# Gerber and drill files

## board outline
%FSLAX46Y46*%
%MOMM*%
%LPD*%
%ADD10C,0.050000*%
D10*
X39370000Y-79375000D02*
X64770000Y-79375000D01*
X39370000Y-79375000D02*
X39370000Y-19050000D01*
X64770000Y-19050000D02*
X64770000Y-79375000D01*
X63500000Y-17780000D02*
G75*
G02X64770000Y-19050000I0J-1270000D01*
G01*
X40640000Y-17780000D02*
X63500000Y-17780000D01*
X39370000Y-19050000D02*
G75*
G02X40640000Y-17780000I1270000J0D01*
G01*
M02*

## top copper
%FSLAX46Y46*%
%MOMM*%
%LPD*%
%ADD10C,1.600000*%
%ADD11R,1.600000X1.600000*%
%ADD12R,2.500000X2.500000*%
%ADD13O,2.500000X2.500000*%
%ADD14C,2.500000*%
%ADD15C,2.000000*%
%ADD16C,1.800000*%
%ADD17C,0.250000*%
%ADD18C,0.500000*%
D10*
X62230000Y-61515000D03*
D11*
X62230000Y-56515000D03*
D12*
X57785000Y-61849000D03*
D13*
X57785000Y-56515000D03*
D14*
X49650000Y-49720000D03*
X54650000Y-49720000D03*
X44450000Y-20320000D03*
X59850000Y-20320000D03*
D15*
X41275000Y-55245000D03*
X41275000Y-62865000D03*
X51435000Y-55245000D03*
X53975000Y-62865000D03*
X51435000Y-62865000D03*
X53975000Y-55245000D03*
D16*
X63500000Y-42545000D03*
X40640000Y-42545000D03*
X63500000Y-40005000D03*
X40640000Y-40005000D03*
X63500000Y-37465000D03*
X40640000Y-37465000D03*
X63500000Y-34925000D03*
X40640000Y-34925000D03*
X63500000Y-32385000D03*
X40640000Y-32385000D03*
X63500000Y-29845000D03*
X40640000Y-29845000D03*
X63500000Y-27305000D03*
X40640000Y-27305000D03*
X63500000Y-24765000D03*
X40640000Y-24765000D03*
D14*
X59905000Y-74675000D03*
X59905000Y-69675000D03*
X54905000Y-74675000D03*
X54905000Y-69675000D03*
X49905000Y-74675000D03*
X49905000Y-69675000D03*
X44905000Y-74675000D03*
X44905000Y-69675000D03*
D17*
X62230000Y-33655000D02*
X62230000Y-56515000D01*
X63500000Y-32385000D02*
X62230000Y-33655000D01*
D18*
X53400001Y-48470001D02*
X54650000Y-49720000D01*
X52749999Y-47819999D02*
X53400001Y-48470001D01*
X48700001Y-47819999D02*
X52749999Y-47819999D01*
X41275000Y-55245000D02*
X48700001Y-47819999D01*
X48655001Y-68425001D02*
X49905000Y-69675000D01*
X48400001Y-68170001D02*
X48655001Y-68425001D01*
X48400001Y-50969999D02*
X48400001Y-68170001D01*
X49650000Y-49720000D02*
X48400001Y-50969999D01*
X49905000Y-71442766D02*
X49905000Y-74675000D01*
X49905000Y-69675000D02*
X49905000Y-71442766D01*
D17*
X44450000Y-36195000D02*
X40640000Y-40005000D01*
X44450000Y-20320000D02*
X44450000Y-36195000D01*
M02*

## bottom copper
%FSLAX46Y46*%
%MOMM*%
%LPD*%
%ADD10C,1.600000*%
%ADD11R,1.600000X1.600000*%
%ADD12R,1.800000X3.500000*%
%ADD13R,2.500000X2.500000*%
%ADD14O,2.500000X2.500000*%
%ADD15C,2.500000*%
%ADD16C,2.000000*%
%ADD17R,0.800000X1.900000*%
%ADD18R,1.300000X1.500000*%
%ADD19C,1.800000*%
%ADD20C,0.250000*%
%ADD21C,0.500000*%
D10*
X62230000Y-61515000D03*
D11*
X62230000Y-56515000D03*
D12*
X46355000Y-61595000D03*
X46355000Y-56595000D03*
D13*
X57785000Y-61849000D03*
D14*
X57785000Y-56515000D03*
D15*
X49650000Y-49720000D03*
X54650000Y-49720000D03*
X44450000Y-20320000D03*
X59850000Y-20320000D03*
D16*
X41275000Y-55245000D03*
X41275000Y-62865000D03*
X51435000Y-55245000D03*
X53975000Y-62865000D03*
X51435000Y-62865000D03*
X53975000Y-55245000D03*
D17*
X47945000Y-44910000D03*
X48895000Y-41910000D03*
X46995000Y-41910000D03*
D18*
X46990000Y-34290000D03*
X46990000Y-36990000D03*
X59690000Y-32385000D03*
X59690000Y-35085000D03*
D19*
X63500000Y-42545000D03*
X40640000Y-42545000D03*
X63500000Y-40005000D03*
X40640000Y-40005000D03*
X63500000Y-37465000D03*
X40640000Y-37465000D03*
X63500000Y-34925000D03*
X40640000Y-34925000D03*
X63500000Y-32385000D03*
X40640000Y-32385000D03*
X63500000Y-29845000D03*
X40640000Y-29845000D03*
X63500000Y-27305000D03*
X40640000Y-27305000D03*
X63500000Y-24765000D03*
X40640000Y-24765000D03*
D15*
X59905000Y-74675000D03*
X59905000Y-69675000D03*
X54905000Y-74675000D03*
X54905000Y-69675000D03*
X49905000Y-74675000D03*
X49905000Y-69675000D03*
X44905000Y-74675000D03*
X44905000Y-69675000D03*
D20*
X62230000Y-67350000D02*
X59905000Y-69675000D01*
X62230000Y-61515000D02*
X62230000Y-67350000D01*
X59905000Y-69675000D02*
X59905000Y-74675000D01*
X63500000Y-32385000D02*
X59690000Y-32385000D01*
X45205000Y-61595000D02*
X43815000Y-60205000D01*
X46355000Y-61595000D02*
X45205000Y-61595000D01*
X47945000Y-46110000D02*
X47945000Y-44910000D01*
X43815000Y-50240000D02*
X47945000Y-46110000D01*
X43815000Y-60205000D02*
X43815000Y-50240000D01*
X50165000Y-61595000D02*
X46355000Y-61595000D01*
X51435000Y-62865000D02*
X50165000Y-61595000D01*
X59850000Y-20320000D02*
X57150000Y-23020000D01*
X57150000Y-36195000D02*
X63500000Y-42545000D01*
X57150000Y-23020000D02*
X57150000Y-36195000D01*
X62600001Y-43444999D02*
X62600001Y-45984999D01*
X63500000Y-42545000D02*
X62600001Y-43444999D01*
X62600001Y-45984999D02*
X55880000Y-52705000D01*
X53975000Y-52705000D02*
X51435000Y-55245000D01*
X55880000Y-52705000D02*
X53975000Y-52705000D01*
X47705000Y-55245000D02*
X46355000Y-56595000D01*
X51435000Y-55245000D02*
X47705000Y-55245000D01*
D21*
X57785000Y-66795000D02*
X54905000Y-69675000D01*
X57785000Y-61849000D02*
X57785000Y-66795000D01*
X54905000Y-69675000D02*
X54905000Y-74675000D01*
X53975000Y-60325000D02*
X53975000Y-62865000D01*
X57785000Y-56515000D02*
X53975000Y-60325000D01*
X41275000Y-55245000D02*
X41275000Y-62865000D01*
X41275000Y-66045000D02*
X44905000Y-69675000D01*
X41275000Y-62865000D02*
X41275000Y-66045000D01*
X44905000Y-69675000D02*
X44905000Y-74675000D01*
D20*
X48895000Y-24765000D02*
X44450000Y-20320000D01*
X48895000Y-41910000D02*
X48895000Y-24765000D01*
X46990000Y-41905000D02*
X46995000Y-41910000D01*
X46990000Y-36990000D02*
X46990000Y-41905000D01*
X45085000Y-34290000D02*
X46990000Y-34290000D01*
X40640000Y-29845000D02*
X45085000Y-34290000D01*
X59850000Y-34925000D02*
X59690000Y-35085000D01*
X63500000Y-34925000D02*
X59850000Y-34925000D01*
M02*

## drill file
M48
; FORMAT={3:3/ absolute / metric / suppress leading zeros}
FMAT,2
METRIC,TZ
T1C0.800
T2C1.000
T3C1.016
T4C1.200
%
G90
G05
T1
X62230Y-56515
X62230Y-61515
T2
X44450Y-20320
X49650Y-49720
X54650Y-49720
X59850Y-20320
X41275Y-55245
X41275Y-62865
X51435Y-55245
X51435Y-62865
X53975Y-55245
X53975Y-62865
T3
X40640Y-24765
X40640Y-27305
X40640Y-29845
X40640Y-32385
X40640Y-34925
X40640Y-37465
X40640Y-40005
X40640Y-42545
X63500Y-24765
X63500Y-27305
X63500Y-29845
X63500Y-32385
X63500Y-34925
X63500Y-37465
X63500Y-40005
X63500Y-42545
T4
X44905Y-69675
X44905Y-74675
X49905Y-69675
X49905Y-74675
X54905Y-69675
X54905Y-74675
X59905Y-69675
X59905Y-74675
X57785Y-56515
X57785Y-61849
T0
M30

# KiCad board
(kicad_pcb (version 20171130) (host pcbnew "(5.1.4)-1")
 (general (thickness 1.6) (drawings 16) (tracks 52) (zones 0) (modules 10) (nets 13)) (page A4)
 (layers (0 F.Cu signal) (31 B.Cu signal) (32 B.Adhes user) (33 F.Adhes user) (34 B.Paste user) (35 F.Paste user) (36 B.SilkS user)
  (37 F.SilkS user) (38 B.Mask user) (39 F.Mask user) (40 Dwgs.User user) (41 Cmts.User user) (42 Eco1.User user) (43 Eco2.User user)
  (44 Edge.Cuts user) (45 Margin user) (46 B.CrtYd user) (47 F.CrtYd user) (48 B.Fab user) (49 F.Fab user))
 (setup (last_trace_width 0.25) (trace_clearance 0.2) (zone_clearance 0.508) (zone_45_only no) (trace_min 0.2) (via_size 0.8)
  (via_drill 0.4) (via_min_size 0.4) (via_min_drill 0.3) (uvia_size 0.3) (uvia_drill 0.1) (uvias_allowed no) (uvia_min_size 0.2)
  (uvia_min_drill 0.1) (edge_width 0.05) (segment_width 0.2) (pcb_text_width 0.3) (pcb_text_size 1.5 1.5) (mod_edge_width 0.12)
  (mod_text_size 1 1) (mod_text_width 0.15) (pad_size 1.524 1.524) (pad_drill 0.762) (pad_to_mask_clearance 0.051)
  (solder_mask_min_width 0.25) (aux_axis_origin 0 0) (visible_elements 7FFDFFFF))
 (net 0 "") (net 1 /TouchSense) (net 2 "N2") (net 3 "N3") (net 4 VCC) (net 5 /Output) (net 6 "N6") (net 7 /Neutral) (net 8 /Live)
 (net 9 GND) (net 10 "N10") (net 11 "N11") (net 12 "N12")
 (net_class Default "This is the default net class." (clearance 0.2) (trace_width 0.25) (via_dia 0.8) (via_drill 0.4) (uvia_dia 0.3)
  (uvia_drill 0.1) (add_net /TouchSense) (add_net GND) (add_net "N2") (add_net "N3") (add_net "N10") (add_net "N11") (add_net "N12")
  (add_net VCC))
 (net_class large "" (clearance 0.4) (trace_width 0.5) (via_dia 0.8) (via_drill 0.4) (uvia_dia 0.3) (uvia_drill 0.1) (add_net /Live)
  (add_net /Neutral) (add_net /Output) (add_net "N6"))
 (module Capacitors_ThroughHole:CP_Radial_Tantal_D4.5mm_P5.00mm (layer F.Cu) (at 62.23 56.515 270)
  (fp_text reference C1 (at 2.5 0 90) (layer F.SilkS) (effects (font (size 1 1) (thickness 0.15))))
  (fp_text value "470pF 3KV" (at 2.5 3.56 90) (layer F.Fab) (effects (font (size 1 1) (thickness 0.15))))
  (pad 2 thru_hole circle (at 5 0 270) (size 1.6 1.6) (drill 0.8) (layers *.Cu *.Mask) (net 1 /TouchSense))
  (pad 1 thru_hole rect (at 0 0 270) (size 1.6 1.6) (drill 0.8) (layers *.Cu *.Mask) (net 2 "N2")))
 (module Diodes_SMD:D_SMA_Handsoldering (layer B.Cu) (at 46.355 59.095 270)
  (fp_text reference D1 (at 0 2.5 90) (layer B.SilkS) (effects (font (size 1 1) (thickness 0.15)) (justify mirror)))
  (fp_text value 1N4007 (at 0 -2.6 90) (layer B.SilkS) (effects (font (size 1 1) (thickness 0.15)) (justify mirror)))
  (pad 2 smd rect (at 2.5 0 270) (size 3.5 1.8) (layers B.Cu B.Paste B.Mask) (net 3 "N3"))
  (pad 1 smd rect (at -2.5 0 270) (size 3.5 1.8) (layers B.Cu B.Paste B.Mask) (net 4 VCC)))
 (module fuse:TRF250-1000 (layer F.Cu) (at 57.785 59.182 180)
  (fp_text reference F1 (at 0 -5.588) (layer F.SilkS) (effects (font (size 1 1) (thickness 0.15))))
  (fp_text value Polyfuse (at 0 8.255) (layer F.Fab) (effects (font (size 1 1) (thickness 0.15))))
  (pad 1 thru_hole rect (at 0 -2.667 180) (size 2.5 2.5) (drill 1.2) (layers *.Cu *.Mask) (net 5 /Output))
  (pad 2 thru_hole oval (at 0 2.667 180) (size 2.5 2.5) (drill 1.2) (layers *.Cu *.Mask) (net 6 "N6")))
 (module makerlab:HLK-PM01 (layer F.Cu) (at 52.15 35.02 90)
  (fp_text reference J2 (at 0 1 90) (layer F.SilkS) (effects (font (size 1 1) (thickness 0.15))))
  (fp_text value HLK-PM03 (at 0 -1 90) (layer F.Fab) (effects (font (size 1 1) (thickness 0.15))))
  (pad 1 thru_hole circle (at -14.7 -2.5 90) (size 2.5 2.5) (drill 1) (layers *.Cu *.Mask F.SilkS) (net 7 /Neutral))
  (pad 2 thru_hole circle (at -14.7 2.5 90) (size 2.5 2.5) (drill 1) (layers *.Cu *.Mask F.SilkS) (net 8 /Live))
  (pad 3 thru_hole circle (at 14.7 -7.7 90) (size 2.5 2.5) (drill 1) (layers *.Cu *.Mask F.SilkS) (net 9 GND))
  (pad 4 thru_hole circle (at 14.7 7.7 90) (size 2.5 2.5) (drill 1) (layers *.Cu *.Mask F.SilkS) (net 4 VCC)))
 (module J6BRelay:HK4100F (layer F.Cu) (at 41.275 55.245)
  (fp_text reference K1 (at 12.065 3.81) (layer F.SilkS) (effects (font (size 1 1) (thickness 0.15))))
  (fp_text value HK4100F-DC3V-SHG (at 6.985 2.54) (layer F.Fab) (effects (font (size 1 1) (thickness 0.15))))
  (pad 11 thru_hole circle (at 0 0) (size 2 2) (drill 1) (layers *.Cu *.Mask) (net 8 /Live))
  (pad 11 thru_hole circle (at 0 7.62) (size 2 2) (drill 1) (layers *.Cu *.Mask) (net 8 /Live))
  (pad A1 thru_hole circle (at 10.16 0) (size 2 2) (drill 1) (layers *.Cu *.Mask) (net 4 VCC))
  (pad 14 thru_hole circle (at 12.7 7.62) (size 2 2) (drill 1) (layers *.Cu *.Mask) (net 6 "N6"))
  (pad A2 thru_hole circle (at 10.16 7.62) (size 2 2) (drill 1) (layers *.Cu *.Mask) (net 3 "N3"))
  (pad 12 thru_hole circle (at 12.7 0) (size 2 2) (drill 1) (layers *.Cu *.Mask)))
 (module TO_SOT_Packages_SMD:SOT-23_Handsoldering (layer B.Cu) (at 47.945 43.41 270)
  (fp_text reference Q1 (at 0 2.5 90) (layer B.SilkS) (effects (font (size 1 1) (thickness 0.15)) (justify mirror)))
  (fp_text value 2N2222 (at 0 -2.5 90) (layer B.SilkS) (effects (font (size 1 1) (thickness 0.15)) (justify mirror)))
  (pad 3 smd rect (at 1.5 0 270) (size 1.9 0.8) (layers B.Cu B.Paste B.Mask) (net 3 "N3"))
  (pad 2 smd rect (at -1.5 -0.95 270) (size 1.9 0.8) (layers B.Cu B.Paste B.Mask) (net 9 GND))
  (pad 1 smd rect (at -1.5 0.95 270) (size 1.9 0.8) (layers B.Cu B.Paste B.Mask) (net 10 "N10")))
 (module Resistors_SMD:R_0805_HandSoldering (layer B.Cu) (at 46.99 35.64 90)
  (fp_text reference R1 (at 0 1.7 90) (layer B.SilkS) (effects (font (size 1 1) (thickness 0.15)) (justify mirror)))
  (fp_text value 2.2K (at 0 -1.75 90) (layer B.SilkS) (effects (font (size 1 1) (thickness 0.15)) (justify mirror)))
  (pad 2 smd rect (at 1.35 0 90) (size 1.5 1.3) (layers B.Cu B.Paste B.Mask) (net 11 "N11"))
  (pad 1 smd rect (at -1.35 0 90) (size 1.5 1.3) (layers B.Cu B.Paste B.Mask) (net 10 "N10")))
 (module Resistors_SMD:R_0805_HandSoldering (layer B.Cu) (at 59.69 33.735 270)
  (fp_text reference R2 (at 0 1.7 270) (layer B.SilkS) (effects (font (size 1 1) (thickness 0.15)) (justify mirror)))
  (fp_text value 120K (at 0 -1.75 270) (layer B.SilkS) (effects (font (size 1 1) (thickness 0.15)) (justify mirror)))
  (pad 1 smd rect (at -1.35 0 270) (size 1.5 1.3) (layers B.Cu B.Paste B.Mask) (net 2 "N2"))
  (pad 2 smd rect (at 1.35 0 270) (size 1.5 1.3) (layers B.Cu B.Paste B.Mask) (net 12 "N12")))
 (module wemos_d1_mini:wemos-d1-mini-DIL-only (layer B.Cu) (at 52.07 33.655 90)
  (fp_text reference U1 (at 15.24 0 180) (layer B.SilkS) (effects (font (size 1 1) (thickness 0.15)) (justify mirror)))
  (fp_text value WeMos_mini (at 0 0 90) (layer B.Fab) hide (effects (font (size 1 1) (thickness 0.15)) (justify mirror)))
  (pad 16 thru_hole circle (at -8.89 11.43 90) (size 1.8 1.8) (drill 1.016) (layers *.Cu *.Mask) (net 4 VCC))
  (pad 1 thru_hole circle (at -8.89 -11.43 90) (size 1.8 1.8) (drill 1.016) (layers *.Cu *.Mask))
  (pad 15 thru_hole circle (at -6.35 11.43 90) (size 1.8 1.8) (drill 1.016) (layers *.Cu *.Mask))
  (pad 2 thru_hole circle (at -6.35 -11.43 90) (size 1.8 1.8) (drill 1.016) (layers *.Cu *.Mask) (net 9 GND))
  (pad 14 thru_hole circle (at -3.81 11.43 90) (size 1.8 1.8) (drill 1.016) (layers *.Cu *.Mask))
  (pad 3 thru_hole circle (at -3.81 -11.43 90) (size 1.8 1.8) (drill 1.016) (layers *.Cu *.Mask))
  (pad 13 thru_hole circle (at -1.27 11.43 90) (size 1.8 1.8) (drill 1.016) (layers *.Cu *.Mask) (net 12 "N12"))
  (pad 4 thru_hole circle (at -1.27 -11.43 90) (size 1.8 1.8) (drill 1.016) (layers *.Cu *.Mask))
  (pad 12 thru_hole circle (at 1.27 11.43 90) (size 1.8 1.8) (drill 1.016) (layers *.Cu *.Mask) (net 2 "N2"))
  (pad 5 thru_hole circle (at 1.27 -11.43 90) (size 1.8 1.8) (drill 1.016) (layers *.Cu *.Mask))
  (pad 11 thru_hole circle (at 3.81 11.43 90) (size 1.8 1.8) (drill 1.016) (layers *.Cu *.Mask))
  (pad 6 thru_hole circle (at 3.81 -11.43 90) (size 1.8 1.8) (drill 1.016) (layers *.Cu *.Mask) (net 11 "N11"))
  (pad 10 thru_hole circle (at 6.35 11.43 90) (size 1.8 1.8) (drill 1.016) (layers *.Cu *.Mask))
  (pad 7 thru_hole circle (at 6.35 -11.43 90) (size 1.8 1.8) (drill 1.016) (layers *.Cu *.Mask))
  (pad 9 thru_hole circle (at 8.89 11.43 90) (size 1.8 1.8) (drill 1.016) (layers *.Cu *.Mask))
  (pad 8 thru_hole circle (at 8.89 -11.43 90) (size 1.8 1.8) (drill 1.016) (layers *.Cu *.Mask)))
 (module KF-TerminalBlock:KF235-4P (layer F.Cu) (at 52.705 79.375)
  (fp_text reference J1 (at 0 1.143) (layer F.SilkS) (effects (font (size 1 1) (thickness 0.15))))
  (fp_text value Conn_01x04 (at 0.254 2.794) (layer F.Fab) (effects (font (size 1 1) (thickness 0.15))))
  (pad 1 thru_hole circle (at 7.2 -4.7) (size 2.5 2.5) (drill 1.2) (layers *.Cu *.Mask) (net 1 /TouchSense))
  (pad 1 thru_hole circle (at 7.2 -9.7) (size 2.5 2.5) (drill 1.2) (layers *.Cu *.Mask) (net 1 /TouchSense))
  (pad 2 thru_hole circle (at 2.2 -4.7) (size 2.5 2.5) (drill 1.2) (layers *.Cu *.Mask) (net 5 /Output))
  (pad 2 thru_hole circle (at 2.2 -9.7) (size 2.5 2.5) (drill 1.2) (layers *.Cu *.Mask) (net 5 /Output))
  (pad 3 thru_hole circle (at -2.8 -4.7) (size 2.5 2.5) (drill 1.2) (layers *.Cu *.Mask) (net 7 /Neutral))
  (pad 3 thru_hole circle (at -2.8 -9.7) (size 2.5 2.5) (drill 1.2) (layers *.Cu *.Mask) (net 7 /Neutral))
  (pad 4 thru_hole circle (at -7.8 -4.7) (size 2.5 2.5) (drill 1.2) (layers *.Cu *.Mask) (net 8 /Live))
  (pad 4 thru_hole circle (at -7.8 -9.7) (size 2.5 2.5) (drill 1.2) (layers *.Cu *.Mask) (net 8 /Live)))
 (gr_line (start 39.37 79.375) (end 64.77 79.375) (layer Edge.Cuts) (width 0.05))
 (gr_line (start 39.37 79.375) (end 39.37 19.05) (layer Edge.Cuts) (width 0.05))
 (gr_line (start 64.77 19.05) (end 64.77 79.375) (layer Edge.Cuts) (width 0.05))
 (gr_arc (start 63.5 19.05) (end 64.77 19.05) (angle -90) (layer Edge.Cuts) (width 0.05))
 (gr_line (start 40.64 17.78) (end 63.5 17.78) (layer Edge.Cuts) (width 0.05))
 (gr_arc (start 40.64 19.05) (end 40.64 17.78) (angle -90) (layer Edge.Cuts) (width 0.05))
 (segment (start 62.23 67.35) (end 59.905 69.675) (width 0.25) (layer B.Cu) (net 1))
 (segment (start 62.23 61.515) (end 62.23 67.35) (width 0.25) (layer B.Cu) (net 1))
 (segment (start 59.905 69.675) (end 59.905 74.675) (width 0.25) (layer B.Cu) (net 1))
 (segment (start 63.5 32.385) (end 59.69 32.385) (width 0.25) (layer B.Cu) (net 2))
 (segment (start 62.23 33.655) (end 62.23 56.515) (width 0.25) (layer F.Cu) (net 2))
 (segment (start 63.5 32.385) (end 62.23 33.655) (width 0.25) (layer F.Cu) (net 2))
 (segment (start 45.205 61.595) (end 43.815 60.205) (width 0.25) (layer B.Cu) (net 3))
 (segment (start 46.355 61.595) (end 45.205 61.595) (width 0.25) (layer B.Cu) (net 3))
 (segment (start 47.945 46.11) (end 47.945 44.91) (width 0.25) (layer B.Cu) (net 3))
 (segment (start 43.815 50.24) (end 47.945 46.11) (width 0.25) (layer B.Cu) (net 3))
 (segment (start 43.815 60.205) (end 43.815 50.24) (width 0.25) (layer B.Cu) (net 3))
 (segment (start 50.165 61.595) (end 46.355 61.595) (width 0.25) (layer B.Cu) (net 3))
 (segment (start 51.435 62.865) (end 50.165 61.595) (width 0.25) (layer B.Cu) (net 3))
 (segment (start 59.85 20.32) (end 57.15 23.02) (width 0.25) (layer B.Cu) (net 4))
 (segment (start 57.15 36.195) (end 63.5 42.545) (width 0.25) (layer B.Cu) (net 4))
 (segment (start 57.15 23.02) (end 57.15 36.195) (width 0.25) (layer B.Cu) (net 4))
 (segment (start 62.600001 43.444999) (end 62.600001 45.984999) (width 0.25) (layer B.Cu) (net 4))
 (segment (start 63.5 42.545) (end 62.600001 43.444999) (width 0.25) (layer B.Cu) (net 4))
 (segment (start 62.600001 45.984999) (end 55.88 52.705) (width 0.25) (layer B.Cu) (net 4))
 (segment (start 53.975 52.705) (end 51.435 55.245) (width 0.25) (layer B.Cu) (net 4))
 (segment (start 55.88 52.705) (end 53.975 52.705) (width 0.25) (layer B.Cu) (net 4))
 (segment (start 47.705 55.245) (end 46.355 56.595) (width 0.25) (layer B.Cu) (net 4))
 (segment (start 51.435 55.245) (end 47.705 55.245) (width 0.25) (layer B.Cu) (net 4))
 (segment (start 57.785 66.795) (end 54.905 69.675) (width 0.5) (layer B.Cu) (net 5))
 (segment (start 57.785 61.849) (end 57.785 66.795) (width 0.5) (layer B.Cu) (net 5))
 (segment (start 54.905 69.675) (end 54.905 74.675) (width 0.5) (layer B.Cu) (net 5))
 (segment (start 53.975 60.325) (end 53.975 62.865) (width 0.5) (layer B.Cu) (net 6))
 (segment (start 57.785 56.515) (end 53.975 60.325) (width 0.5) (layer B.Cu) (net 6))
 (segment (start 53.400001 48.470001) (end 54.65 49.72) (width 0.5) (layer F.Cu) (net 8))
 (segment (start 52.749999 47.819999) (end 53.400001 48.470001) (width 0.5) (layer F.Cu) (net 8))
 (segment (start 48.700001 47.819999) (end 52.749999 47.819999) (width 0.5) (layer F.Cu) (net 8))
 (segment (start 41.275 55.245) (end 48.700001 47.819999) (width 0.5) (layer F.Cu) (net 8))
 (segment (start 41.275 55.245) (end 41.275 62.865) (width 0.5) (layer B.Cu) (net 8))
 (segment (start 41.275 66.045) (end 44.905 69.675) (width 0.5) (layer B.Cu) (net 8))
 (segment (start 41.275 62.865) (end 41.275 66.045) (width 0.5) (layer B.Cu) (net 8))
 (segment (start 44.905 69.675) (end 44.905 74.675) (width 0.5) (layer B.Cu) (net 8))
 (segment (start 48.655001 68.425001) (end 49.905 69.675) (width 0.5) (layer F.Cu) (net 7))
 (segment (start 48.400001 68.170001) (end 48.655001 68.425001) (width 0.5) (layer F.Cu) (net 7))
 (segment (start 48.400001 50.969999) (end 48.400001 68.170001) (width 0.5) (layer F.Cu) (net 7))
 (segment (start 49.65 49.72) (end 48.400001 50.969999) (width 0.5) (layer F.Cu) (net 7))
 (segment (start 49.905 71.442766) (end 49.905 74.675) (width 0.5) (layer F.Cu) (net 7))
 (segment (start 49.905 69.675) (end 49.905 71.442766) (width 0.5) (layer F.Cu) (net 7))
 (segment (start 48.895 24.765) (end 44.45 20.32) (width 0.25) (layer B.Cu) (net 9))
 (segment (start 48.895 41.91) (end 48.895 24.765) (width 0.25) (layer B.Cu) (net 9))
 (segment (start 44.45 36.195) (end 40.64 40.005) (width 0.25) (layer F.Cu) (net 9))
 (segment (start 44.45 20.32) (end 44.45 36.195) (width 0.25) (layer F.Cu) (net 9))
 (segment (start 46.99 41.905) (end 46.995 41.91) (width 0.25) (layer B.Cu) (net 10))
 (segment (start 46.99 36.99) (end 46.99 41.905) (width 0.25) (layer B.Cu) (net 10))
 (segment (start 45.085 34.29) (end 46.99 34.29) (width 0.25) (layer B.Cu) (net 11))
 (segment (start 40.64 29.845) (end 45.085 34.29) (width 0.25) (layer B.Cu) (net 11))
 (segment (start 59.85 34.925) (end 59.69 35.085) (width 0.25) (layer B.Cu) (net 12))
 (segment (start 63.5 34.925) (end 59.85 34.925) (width 0.25) (layer B.Cu) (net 12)))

